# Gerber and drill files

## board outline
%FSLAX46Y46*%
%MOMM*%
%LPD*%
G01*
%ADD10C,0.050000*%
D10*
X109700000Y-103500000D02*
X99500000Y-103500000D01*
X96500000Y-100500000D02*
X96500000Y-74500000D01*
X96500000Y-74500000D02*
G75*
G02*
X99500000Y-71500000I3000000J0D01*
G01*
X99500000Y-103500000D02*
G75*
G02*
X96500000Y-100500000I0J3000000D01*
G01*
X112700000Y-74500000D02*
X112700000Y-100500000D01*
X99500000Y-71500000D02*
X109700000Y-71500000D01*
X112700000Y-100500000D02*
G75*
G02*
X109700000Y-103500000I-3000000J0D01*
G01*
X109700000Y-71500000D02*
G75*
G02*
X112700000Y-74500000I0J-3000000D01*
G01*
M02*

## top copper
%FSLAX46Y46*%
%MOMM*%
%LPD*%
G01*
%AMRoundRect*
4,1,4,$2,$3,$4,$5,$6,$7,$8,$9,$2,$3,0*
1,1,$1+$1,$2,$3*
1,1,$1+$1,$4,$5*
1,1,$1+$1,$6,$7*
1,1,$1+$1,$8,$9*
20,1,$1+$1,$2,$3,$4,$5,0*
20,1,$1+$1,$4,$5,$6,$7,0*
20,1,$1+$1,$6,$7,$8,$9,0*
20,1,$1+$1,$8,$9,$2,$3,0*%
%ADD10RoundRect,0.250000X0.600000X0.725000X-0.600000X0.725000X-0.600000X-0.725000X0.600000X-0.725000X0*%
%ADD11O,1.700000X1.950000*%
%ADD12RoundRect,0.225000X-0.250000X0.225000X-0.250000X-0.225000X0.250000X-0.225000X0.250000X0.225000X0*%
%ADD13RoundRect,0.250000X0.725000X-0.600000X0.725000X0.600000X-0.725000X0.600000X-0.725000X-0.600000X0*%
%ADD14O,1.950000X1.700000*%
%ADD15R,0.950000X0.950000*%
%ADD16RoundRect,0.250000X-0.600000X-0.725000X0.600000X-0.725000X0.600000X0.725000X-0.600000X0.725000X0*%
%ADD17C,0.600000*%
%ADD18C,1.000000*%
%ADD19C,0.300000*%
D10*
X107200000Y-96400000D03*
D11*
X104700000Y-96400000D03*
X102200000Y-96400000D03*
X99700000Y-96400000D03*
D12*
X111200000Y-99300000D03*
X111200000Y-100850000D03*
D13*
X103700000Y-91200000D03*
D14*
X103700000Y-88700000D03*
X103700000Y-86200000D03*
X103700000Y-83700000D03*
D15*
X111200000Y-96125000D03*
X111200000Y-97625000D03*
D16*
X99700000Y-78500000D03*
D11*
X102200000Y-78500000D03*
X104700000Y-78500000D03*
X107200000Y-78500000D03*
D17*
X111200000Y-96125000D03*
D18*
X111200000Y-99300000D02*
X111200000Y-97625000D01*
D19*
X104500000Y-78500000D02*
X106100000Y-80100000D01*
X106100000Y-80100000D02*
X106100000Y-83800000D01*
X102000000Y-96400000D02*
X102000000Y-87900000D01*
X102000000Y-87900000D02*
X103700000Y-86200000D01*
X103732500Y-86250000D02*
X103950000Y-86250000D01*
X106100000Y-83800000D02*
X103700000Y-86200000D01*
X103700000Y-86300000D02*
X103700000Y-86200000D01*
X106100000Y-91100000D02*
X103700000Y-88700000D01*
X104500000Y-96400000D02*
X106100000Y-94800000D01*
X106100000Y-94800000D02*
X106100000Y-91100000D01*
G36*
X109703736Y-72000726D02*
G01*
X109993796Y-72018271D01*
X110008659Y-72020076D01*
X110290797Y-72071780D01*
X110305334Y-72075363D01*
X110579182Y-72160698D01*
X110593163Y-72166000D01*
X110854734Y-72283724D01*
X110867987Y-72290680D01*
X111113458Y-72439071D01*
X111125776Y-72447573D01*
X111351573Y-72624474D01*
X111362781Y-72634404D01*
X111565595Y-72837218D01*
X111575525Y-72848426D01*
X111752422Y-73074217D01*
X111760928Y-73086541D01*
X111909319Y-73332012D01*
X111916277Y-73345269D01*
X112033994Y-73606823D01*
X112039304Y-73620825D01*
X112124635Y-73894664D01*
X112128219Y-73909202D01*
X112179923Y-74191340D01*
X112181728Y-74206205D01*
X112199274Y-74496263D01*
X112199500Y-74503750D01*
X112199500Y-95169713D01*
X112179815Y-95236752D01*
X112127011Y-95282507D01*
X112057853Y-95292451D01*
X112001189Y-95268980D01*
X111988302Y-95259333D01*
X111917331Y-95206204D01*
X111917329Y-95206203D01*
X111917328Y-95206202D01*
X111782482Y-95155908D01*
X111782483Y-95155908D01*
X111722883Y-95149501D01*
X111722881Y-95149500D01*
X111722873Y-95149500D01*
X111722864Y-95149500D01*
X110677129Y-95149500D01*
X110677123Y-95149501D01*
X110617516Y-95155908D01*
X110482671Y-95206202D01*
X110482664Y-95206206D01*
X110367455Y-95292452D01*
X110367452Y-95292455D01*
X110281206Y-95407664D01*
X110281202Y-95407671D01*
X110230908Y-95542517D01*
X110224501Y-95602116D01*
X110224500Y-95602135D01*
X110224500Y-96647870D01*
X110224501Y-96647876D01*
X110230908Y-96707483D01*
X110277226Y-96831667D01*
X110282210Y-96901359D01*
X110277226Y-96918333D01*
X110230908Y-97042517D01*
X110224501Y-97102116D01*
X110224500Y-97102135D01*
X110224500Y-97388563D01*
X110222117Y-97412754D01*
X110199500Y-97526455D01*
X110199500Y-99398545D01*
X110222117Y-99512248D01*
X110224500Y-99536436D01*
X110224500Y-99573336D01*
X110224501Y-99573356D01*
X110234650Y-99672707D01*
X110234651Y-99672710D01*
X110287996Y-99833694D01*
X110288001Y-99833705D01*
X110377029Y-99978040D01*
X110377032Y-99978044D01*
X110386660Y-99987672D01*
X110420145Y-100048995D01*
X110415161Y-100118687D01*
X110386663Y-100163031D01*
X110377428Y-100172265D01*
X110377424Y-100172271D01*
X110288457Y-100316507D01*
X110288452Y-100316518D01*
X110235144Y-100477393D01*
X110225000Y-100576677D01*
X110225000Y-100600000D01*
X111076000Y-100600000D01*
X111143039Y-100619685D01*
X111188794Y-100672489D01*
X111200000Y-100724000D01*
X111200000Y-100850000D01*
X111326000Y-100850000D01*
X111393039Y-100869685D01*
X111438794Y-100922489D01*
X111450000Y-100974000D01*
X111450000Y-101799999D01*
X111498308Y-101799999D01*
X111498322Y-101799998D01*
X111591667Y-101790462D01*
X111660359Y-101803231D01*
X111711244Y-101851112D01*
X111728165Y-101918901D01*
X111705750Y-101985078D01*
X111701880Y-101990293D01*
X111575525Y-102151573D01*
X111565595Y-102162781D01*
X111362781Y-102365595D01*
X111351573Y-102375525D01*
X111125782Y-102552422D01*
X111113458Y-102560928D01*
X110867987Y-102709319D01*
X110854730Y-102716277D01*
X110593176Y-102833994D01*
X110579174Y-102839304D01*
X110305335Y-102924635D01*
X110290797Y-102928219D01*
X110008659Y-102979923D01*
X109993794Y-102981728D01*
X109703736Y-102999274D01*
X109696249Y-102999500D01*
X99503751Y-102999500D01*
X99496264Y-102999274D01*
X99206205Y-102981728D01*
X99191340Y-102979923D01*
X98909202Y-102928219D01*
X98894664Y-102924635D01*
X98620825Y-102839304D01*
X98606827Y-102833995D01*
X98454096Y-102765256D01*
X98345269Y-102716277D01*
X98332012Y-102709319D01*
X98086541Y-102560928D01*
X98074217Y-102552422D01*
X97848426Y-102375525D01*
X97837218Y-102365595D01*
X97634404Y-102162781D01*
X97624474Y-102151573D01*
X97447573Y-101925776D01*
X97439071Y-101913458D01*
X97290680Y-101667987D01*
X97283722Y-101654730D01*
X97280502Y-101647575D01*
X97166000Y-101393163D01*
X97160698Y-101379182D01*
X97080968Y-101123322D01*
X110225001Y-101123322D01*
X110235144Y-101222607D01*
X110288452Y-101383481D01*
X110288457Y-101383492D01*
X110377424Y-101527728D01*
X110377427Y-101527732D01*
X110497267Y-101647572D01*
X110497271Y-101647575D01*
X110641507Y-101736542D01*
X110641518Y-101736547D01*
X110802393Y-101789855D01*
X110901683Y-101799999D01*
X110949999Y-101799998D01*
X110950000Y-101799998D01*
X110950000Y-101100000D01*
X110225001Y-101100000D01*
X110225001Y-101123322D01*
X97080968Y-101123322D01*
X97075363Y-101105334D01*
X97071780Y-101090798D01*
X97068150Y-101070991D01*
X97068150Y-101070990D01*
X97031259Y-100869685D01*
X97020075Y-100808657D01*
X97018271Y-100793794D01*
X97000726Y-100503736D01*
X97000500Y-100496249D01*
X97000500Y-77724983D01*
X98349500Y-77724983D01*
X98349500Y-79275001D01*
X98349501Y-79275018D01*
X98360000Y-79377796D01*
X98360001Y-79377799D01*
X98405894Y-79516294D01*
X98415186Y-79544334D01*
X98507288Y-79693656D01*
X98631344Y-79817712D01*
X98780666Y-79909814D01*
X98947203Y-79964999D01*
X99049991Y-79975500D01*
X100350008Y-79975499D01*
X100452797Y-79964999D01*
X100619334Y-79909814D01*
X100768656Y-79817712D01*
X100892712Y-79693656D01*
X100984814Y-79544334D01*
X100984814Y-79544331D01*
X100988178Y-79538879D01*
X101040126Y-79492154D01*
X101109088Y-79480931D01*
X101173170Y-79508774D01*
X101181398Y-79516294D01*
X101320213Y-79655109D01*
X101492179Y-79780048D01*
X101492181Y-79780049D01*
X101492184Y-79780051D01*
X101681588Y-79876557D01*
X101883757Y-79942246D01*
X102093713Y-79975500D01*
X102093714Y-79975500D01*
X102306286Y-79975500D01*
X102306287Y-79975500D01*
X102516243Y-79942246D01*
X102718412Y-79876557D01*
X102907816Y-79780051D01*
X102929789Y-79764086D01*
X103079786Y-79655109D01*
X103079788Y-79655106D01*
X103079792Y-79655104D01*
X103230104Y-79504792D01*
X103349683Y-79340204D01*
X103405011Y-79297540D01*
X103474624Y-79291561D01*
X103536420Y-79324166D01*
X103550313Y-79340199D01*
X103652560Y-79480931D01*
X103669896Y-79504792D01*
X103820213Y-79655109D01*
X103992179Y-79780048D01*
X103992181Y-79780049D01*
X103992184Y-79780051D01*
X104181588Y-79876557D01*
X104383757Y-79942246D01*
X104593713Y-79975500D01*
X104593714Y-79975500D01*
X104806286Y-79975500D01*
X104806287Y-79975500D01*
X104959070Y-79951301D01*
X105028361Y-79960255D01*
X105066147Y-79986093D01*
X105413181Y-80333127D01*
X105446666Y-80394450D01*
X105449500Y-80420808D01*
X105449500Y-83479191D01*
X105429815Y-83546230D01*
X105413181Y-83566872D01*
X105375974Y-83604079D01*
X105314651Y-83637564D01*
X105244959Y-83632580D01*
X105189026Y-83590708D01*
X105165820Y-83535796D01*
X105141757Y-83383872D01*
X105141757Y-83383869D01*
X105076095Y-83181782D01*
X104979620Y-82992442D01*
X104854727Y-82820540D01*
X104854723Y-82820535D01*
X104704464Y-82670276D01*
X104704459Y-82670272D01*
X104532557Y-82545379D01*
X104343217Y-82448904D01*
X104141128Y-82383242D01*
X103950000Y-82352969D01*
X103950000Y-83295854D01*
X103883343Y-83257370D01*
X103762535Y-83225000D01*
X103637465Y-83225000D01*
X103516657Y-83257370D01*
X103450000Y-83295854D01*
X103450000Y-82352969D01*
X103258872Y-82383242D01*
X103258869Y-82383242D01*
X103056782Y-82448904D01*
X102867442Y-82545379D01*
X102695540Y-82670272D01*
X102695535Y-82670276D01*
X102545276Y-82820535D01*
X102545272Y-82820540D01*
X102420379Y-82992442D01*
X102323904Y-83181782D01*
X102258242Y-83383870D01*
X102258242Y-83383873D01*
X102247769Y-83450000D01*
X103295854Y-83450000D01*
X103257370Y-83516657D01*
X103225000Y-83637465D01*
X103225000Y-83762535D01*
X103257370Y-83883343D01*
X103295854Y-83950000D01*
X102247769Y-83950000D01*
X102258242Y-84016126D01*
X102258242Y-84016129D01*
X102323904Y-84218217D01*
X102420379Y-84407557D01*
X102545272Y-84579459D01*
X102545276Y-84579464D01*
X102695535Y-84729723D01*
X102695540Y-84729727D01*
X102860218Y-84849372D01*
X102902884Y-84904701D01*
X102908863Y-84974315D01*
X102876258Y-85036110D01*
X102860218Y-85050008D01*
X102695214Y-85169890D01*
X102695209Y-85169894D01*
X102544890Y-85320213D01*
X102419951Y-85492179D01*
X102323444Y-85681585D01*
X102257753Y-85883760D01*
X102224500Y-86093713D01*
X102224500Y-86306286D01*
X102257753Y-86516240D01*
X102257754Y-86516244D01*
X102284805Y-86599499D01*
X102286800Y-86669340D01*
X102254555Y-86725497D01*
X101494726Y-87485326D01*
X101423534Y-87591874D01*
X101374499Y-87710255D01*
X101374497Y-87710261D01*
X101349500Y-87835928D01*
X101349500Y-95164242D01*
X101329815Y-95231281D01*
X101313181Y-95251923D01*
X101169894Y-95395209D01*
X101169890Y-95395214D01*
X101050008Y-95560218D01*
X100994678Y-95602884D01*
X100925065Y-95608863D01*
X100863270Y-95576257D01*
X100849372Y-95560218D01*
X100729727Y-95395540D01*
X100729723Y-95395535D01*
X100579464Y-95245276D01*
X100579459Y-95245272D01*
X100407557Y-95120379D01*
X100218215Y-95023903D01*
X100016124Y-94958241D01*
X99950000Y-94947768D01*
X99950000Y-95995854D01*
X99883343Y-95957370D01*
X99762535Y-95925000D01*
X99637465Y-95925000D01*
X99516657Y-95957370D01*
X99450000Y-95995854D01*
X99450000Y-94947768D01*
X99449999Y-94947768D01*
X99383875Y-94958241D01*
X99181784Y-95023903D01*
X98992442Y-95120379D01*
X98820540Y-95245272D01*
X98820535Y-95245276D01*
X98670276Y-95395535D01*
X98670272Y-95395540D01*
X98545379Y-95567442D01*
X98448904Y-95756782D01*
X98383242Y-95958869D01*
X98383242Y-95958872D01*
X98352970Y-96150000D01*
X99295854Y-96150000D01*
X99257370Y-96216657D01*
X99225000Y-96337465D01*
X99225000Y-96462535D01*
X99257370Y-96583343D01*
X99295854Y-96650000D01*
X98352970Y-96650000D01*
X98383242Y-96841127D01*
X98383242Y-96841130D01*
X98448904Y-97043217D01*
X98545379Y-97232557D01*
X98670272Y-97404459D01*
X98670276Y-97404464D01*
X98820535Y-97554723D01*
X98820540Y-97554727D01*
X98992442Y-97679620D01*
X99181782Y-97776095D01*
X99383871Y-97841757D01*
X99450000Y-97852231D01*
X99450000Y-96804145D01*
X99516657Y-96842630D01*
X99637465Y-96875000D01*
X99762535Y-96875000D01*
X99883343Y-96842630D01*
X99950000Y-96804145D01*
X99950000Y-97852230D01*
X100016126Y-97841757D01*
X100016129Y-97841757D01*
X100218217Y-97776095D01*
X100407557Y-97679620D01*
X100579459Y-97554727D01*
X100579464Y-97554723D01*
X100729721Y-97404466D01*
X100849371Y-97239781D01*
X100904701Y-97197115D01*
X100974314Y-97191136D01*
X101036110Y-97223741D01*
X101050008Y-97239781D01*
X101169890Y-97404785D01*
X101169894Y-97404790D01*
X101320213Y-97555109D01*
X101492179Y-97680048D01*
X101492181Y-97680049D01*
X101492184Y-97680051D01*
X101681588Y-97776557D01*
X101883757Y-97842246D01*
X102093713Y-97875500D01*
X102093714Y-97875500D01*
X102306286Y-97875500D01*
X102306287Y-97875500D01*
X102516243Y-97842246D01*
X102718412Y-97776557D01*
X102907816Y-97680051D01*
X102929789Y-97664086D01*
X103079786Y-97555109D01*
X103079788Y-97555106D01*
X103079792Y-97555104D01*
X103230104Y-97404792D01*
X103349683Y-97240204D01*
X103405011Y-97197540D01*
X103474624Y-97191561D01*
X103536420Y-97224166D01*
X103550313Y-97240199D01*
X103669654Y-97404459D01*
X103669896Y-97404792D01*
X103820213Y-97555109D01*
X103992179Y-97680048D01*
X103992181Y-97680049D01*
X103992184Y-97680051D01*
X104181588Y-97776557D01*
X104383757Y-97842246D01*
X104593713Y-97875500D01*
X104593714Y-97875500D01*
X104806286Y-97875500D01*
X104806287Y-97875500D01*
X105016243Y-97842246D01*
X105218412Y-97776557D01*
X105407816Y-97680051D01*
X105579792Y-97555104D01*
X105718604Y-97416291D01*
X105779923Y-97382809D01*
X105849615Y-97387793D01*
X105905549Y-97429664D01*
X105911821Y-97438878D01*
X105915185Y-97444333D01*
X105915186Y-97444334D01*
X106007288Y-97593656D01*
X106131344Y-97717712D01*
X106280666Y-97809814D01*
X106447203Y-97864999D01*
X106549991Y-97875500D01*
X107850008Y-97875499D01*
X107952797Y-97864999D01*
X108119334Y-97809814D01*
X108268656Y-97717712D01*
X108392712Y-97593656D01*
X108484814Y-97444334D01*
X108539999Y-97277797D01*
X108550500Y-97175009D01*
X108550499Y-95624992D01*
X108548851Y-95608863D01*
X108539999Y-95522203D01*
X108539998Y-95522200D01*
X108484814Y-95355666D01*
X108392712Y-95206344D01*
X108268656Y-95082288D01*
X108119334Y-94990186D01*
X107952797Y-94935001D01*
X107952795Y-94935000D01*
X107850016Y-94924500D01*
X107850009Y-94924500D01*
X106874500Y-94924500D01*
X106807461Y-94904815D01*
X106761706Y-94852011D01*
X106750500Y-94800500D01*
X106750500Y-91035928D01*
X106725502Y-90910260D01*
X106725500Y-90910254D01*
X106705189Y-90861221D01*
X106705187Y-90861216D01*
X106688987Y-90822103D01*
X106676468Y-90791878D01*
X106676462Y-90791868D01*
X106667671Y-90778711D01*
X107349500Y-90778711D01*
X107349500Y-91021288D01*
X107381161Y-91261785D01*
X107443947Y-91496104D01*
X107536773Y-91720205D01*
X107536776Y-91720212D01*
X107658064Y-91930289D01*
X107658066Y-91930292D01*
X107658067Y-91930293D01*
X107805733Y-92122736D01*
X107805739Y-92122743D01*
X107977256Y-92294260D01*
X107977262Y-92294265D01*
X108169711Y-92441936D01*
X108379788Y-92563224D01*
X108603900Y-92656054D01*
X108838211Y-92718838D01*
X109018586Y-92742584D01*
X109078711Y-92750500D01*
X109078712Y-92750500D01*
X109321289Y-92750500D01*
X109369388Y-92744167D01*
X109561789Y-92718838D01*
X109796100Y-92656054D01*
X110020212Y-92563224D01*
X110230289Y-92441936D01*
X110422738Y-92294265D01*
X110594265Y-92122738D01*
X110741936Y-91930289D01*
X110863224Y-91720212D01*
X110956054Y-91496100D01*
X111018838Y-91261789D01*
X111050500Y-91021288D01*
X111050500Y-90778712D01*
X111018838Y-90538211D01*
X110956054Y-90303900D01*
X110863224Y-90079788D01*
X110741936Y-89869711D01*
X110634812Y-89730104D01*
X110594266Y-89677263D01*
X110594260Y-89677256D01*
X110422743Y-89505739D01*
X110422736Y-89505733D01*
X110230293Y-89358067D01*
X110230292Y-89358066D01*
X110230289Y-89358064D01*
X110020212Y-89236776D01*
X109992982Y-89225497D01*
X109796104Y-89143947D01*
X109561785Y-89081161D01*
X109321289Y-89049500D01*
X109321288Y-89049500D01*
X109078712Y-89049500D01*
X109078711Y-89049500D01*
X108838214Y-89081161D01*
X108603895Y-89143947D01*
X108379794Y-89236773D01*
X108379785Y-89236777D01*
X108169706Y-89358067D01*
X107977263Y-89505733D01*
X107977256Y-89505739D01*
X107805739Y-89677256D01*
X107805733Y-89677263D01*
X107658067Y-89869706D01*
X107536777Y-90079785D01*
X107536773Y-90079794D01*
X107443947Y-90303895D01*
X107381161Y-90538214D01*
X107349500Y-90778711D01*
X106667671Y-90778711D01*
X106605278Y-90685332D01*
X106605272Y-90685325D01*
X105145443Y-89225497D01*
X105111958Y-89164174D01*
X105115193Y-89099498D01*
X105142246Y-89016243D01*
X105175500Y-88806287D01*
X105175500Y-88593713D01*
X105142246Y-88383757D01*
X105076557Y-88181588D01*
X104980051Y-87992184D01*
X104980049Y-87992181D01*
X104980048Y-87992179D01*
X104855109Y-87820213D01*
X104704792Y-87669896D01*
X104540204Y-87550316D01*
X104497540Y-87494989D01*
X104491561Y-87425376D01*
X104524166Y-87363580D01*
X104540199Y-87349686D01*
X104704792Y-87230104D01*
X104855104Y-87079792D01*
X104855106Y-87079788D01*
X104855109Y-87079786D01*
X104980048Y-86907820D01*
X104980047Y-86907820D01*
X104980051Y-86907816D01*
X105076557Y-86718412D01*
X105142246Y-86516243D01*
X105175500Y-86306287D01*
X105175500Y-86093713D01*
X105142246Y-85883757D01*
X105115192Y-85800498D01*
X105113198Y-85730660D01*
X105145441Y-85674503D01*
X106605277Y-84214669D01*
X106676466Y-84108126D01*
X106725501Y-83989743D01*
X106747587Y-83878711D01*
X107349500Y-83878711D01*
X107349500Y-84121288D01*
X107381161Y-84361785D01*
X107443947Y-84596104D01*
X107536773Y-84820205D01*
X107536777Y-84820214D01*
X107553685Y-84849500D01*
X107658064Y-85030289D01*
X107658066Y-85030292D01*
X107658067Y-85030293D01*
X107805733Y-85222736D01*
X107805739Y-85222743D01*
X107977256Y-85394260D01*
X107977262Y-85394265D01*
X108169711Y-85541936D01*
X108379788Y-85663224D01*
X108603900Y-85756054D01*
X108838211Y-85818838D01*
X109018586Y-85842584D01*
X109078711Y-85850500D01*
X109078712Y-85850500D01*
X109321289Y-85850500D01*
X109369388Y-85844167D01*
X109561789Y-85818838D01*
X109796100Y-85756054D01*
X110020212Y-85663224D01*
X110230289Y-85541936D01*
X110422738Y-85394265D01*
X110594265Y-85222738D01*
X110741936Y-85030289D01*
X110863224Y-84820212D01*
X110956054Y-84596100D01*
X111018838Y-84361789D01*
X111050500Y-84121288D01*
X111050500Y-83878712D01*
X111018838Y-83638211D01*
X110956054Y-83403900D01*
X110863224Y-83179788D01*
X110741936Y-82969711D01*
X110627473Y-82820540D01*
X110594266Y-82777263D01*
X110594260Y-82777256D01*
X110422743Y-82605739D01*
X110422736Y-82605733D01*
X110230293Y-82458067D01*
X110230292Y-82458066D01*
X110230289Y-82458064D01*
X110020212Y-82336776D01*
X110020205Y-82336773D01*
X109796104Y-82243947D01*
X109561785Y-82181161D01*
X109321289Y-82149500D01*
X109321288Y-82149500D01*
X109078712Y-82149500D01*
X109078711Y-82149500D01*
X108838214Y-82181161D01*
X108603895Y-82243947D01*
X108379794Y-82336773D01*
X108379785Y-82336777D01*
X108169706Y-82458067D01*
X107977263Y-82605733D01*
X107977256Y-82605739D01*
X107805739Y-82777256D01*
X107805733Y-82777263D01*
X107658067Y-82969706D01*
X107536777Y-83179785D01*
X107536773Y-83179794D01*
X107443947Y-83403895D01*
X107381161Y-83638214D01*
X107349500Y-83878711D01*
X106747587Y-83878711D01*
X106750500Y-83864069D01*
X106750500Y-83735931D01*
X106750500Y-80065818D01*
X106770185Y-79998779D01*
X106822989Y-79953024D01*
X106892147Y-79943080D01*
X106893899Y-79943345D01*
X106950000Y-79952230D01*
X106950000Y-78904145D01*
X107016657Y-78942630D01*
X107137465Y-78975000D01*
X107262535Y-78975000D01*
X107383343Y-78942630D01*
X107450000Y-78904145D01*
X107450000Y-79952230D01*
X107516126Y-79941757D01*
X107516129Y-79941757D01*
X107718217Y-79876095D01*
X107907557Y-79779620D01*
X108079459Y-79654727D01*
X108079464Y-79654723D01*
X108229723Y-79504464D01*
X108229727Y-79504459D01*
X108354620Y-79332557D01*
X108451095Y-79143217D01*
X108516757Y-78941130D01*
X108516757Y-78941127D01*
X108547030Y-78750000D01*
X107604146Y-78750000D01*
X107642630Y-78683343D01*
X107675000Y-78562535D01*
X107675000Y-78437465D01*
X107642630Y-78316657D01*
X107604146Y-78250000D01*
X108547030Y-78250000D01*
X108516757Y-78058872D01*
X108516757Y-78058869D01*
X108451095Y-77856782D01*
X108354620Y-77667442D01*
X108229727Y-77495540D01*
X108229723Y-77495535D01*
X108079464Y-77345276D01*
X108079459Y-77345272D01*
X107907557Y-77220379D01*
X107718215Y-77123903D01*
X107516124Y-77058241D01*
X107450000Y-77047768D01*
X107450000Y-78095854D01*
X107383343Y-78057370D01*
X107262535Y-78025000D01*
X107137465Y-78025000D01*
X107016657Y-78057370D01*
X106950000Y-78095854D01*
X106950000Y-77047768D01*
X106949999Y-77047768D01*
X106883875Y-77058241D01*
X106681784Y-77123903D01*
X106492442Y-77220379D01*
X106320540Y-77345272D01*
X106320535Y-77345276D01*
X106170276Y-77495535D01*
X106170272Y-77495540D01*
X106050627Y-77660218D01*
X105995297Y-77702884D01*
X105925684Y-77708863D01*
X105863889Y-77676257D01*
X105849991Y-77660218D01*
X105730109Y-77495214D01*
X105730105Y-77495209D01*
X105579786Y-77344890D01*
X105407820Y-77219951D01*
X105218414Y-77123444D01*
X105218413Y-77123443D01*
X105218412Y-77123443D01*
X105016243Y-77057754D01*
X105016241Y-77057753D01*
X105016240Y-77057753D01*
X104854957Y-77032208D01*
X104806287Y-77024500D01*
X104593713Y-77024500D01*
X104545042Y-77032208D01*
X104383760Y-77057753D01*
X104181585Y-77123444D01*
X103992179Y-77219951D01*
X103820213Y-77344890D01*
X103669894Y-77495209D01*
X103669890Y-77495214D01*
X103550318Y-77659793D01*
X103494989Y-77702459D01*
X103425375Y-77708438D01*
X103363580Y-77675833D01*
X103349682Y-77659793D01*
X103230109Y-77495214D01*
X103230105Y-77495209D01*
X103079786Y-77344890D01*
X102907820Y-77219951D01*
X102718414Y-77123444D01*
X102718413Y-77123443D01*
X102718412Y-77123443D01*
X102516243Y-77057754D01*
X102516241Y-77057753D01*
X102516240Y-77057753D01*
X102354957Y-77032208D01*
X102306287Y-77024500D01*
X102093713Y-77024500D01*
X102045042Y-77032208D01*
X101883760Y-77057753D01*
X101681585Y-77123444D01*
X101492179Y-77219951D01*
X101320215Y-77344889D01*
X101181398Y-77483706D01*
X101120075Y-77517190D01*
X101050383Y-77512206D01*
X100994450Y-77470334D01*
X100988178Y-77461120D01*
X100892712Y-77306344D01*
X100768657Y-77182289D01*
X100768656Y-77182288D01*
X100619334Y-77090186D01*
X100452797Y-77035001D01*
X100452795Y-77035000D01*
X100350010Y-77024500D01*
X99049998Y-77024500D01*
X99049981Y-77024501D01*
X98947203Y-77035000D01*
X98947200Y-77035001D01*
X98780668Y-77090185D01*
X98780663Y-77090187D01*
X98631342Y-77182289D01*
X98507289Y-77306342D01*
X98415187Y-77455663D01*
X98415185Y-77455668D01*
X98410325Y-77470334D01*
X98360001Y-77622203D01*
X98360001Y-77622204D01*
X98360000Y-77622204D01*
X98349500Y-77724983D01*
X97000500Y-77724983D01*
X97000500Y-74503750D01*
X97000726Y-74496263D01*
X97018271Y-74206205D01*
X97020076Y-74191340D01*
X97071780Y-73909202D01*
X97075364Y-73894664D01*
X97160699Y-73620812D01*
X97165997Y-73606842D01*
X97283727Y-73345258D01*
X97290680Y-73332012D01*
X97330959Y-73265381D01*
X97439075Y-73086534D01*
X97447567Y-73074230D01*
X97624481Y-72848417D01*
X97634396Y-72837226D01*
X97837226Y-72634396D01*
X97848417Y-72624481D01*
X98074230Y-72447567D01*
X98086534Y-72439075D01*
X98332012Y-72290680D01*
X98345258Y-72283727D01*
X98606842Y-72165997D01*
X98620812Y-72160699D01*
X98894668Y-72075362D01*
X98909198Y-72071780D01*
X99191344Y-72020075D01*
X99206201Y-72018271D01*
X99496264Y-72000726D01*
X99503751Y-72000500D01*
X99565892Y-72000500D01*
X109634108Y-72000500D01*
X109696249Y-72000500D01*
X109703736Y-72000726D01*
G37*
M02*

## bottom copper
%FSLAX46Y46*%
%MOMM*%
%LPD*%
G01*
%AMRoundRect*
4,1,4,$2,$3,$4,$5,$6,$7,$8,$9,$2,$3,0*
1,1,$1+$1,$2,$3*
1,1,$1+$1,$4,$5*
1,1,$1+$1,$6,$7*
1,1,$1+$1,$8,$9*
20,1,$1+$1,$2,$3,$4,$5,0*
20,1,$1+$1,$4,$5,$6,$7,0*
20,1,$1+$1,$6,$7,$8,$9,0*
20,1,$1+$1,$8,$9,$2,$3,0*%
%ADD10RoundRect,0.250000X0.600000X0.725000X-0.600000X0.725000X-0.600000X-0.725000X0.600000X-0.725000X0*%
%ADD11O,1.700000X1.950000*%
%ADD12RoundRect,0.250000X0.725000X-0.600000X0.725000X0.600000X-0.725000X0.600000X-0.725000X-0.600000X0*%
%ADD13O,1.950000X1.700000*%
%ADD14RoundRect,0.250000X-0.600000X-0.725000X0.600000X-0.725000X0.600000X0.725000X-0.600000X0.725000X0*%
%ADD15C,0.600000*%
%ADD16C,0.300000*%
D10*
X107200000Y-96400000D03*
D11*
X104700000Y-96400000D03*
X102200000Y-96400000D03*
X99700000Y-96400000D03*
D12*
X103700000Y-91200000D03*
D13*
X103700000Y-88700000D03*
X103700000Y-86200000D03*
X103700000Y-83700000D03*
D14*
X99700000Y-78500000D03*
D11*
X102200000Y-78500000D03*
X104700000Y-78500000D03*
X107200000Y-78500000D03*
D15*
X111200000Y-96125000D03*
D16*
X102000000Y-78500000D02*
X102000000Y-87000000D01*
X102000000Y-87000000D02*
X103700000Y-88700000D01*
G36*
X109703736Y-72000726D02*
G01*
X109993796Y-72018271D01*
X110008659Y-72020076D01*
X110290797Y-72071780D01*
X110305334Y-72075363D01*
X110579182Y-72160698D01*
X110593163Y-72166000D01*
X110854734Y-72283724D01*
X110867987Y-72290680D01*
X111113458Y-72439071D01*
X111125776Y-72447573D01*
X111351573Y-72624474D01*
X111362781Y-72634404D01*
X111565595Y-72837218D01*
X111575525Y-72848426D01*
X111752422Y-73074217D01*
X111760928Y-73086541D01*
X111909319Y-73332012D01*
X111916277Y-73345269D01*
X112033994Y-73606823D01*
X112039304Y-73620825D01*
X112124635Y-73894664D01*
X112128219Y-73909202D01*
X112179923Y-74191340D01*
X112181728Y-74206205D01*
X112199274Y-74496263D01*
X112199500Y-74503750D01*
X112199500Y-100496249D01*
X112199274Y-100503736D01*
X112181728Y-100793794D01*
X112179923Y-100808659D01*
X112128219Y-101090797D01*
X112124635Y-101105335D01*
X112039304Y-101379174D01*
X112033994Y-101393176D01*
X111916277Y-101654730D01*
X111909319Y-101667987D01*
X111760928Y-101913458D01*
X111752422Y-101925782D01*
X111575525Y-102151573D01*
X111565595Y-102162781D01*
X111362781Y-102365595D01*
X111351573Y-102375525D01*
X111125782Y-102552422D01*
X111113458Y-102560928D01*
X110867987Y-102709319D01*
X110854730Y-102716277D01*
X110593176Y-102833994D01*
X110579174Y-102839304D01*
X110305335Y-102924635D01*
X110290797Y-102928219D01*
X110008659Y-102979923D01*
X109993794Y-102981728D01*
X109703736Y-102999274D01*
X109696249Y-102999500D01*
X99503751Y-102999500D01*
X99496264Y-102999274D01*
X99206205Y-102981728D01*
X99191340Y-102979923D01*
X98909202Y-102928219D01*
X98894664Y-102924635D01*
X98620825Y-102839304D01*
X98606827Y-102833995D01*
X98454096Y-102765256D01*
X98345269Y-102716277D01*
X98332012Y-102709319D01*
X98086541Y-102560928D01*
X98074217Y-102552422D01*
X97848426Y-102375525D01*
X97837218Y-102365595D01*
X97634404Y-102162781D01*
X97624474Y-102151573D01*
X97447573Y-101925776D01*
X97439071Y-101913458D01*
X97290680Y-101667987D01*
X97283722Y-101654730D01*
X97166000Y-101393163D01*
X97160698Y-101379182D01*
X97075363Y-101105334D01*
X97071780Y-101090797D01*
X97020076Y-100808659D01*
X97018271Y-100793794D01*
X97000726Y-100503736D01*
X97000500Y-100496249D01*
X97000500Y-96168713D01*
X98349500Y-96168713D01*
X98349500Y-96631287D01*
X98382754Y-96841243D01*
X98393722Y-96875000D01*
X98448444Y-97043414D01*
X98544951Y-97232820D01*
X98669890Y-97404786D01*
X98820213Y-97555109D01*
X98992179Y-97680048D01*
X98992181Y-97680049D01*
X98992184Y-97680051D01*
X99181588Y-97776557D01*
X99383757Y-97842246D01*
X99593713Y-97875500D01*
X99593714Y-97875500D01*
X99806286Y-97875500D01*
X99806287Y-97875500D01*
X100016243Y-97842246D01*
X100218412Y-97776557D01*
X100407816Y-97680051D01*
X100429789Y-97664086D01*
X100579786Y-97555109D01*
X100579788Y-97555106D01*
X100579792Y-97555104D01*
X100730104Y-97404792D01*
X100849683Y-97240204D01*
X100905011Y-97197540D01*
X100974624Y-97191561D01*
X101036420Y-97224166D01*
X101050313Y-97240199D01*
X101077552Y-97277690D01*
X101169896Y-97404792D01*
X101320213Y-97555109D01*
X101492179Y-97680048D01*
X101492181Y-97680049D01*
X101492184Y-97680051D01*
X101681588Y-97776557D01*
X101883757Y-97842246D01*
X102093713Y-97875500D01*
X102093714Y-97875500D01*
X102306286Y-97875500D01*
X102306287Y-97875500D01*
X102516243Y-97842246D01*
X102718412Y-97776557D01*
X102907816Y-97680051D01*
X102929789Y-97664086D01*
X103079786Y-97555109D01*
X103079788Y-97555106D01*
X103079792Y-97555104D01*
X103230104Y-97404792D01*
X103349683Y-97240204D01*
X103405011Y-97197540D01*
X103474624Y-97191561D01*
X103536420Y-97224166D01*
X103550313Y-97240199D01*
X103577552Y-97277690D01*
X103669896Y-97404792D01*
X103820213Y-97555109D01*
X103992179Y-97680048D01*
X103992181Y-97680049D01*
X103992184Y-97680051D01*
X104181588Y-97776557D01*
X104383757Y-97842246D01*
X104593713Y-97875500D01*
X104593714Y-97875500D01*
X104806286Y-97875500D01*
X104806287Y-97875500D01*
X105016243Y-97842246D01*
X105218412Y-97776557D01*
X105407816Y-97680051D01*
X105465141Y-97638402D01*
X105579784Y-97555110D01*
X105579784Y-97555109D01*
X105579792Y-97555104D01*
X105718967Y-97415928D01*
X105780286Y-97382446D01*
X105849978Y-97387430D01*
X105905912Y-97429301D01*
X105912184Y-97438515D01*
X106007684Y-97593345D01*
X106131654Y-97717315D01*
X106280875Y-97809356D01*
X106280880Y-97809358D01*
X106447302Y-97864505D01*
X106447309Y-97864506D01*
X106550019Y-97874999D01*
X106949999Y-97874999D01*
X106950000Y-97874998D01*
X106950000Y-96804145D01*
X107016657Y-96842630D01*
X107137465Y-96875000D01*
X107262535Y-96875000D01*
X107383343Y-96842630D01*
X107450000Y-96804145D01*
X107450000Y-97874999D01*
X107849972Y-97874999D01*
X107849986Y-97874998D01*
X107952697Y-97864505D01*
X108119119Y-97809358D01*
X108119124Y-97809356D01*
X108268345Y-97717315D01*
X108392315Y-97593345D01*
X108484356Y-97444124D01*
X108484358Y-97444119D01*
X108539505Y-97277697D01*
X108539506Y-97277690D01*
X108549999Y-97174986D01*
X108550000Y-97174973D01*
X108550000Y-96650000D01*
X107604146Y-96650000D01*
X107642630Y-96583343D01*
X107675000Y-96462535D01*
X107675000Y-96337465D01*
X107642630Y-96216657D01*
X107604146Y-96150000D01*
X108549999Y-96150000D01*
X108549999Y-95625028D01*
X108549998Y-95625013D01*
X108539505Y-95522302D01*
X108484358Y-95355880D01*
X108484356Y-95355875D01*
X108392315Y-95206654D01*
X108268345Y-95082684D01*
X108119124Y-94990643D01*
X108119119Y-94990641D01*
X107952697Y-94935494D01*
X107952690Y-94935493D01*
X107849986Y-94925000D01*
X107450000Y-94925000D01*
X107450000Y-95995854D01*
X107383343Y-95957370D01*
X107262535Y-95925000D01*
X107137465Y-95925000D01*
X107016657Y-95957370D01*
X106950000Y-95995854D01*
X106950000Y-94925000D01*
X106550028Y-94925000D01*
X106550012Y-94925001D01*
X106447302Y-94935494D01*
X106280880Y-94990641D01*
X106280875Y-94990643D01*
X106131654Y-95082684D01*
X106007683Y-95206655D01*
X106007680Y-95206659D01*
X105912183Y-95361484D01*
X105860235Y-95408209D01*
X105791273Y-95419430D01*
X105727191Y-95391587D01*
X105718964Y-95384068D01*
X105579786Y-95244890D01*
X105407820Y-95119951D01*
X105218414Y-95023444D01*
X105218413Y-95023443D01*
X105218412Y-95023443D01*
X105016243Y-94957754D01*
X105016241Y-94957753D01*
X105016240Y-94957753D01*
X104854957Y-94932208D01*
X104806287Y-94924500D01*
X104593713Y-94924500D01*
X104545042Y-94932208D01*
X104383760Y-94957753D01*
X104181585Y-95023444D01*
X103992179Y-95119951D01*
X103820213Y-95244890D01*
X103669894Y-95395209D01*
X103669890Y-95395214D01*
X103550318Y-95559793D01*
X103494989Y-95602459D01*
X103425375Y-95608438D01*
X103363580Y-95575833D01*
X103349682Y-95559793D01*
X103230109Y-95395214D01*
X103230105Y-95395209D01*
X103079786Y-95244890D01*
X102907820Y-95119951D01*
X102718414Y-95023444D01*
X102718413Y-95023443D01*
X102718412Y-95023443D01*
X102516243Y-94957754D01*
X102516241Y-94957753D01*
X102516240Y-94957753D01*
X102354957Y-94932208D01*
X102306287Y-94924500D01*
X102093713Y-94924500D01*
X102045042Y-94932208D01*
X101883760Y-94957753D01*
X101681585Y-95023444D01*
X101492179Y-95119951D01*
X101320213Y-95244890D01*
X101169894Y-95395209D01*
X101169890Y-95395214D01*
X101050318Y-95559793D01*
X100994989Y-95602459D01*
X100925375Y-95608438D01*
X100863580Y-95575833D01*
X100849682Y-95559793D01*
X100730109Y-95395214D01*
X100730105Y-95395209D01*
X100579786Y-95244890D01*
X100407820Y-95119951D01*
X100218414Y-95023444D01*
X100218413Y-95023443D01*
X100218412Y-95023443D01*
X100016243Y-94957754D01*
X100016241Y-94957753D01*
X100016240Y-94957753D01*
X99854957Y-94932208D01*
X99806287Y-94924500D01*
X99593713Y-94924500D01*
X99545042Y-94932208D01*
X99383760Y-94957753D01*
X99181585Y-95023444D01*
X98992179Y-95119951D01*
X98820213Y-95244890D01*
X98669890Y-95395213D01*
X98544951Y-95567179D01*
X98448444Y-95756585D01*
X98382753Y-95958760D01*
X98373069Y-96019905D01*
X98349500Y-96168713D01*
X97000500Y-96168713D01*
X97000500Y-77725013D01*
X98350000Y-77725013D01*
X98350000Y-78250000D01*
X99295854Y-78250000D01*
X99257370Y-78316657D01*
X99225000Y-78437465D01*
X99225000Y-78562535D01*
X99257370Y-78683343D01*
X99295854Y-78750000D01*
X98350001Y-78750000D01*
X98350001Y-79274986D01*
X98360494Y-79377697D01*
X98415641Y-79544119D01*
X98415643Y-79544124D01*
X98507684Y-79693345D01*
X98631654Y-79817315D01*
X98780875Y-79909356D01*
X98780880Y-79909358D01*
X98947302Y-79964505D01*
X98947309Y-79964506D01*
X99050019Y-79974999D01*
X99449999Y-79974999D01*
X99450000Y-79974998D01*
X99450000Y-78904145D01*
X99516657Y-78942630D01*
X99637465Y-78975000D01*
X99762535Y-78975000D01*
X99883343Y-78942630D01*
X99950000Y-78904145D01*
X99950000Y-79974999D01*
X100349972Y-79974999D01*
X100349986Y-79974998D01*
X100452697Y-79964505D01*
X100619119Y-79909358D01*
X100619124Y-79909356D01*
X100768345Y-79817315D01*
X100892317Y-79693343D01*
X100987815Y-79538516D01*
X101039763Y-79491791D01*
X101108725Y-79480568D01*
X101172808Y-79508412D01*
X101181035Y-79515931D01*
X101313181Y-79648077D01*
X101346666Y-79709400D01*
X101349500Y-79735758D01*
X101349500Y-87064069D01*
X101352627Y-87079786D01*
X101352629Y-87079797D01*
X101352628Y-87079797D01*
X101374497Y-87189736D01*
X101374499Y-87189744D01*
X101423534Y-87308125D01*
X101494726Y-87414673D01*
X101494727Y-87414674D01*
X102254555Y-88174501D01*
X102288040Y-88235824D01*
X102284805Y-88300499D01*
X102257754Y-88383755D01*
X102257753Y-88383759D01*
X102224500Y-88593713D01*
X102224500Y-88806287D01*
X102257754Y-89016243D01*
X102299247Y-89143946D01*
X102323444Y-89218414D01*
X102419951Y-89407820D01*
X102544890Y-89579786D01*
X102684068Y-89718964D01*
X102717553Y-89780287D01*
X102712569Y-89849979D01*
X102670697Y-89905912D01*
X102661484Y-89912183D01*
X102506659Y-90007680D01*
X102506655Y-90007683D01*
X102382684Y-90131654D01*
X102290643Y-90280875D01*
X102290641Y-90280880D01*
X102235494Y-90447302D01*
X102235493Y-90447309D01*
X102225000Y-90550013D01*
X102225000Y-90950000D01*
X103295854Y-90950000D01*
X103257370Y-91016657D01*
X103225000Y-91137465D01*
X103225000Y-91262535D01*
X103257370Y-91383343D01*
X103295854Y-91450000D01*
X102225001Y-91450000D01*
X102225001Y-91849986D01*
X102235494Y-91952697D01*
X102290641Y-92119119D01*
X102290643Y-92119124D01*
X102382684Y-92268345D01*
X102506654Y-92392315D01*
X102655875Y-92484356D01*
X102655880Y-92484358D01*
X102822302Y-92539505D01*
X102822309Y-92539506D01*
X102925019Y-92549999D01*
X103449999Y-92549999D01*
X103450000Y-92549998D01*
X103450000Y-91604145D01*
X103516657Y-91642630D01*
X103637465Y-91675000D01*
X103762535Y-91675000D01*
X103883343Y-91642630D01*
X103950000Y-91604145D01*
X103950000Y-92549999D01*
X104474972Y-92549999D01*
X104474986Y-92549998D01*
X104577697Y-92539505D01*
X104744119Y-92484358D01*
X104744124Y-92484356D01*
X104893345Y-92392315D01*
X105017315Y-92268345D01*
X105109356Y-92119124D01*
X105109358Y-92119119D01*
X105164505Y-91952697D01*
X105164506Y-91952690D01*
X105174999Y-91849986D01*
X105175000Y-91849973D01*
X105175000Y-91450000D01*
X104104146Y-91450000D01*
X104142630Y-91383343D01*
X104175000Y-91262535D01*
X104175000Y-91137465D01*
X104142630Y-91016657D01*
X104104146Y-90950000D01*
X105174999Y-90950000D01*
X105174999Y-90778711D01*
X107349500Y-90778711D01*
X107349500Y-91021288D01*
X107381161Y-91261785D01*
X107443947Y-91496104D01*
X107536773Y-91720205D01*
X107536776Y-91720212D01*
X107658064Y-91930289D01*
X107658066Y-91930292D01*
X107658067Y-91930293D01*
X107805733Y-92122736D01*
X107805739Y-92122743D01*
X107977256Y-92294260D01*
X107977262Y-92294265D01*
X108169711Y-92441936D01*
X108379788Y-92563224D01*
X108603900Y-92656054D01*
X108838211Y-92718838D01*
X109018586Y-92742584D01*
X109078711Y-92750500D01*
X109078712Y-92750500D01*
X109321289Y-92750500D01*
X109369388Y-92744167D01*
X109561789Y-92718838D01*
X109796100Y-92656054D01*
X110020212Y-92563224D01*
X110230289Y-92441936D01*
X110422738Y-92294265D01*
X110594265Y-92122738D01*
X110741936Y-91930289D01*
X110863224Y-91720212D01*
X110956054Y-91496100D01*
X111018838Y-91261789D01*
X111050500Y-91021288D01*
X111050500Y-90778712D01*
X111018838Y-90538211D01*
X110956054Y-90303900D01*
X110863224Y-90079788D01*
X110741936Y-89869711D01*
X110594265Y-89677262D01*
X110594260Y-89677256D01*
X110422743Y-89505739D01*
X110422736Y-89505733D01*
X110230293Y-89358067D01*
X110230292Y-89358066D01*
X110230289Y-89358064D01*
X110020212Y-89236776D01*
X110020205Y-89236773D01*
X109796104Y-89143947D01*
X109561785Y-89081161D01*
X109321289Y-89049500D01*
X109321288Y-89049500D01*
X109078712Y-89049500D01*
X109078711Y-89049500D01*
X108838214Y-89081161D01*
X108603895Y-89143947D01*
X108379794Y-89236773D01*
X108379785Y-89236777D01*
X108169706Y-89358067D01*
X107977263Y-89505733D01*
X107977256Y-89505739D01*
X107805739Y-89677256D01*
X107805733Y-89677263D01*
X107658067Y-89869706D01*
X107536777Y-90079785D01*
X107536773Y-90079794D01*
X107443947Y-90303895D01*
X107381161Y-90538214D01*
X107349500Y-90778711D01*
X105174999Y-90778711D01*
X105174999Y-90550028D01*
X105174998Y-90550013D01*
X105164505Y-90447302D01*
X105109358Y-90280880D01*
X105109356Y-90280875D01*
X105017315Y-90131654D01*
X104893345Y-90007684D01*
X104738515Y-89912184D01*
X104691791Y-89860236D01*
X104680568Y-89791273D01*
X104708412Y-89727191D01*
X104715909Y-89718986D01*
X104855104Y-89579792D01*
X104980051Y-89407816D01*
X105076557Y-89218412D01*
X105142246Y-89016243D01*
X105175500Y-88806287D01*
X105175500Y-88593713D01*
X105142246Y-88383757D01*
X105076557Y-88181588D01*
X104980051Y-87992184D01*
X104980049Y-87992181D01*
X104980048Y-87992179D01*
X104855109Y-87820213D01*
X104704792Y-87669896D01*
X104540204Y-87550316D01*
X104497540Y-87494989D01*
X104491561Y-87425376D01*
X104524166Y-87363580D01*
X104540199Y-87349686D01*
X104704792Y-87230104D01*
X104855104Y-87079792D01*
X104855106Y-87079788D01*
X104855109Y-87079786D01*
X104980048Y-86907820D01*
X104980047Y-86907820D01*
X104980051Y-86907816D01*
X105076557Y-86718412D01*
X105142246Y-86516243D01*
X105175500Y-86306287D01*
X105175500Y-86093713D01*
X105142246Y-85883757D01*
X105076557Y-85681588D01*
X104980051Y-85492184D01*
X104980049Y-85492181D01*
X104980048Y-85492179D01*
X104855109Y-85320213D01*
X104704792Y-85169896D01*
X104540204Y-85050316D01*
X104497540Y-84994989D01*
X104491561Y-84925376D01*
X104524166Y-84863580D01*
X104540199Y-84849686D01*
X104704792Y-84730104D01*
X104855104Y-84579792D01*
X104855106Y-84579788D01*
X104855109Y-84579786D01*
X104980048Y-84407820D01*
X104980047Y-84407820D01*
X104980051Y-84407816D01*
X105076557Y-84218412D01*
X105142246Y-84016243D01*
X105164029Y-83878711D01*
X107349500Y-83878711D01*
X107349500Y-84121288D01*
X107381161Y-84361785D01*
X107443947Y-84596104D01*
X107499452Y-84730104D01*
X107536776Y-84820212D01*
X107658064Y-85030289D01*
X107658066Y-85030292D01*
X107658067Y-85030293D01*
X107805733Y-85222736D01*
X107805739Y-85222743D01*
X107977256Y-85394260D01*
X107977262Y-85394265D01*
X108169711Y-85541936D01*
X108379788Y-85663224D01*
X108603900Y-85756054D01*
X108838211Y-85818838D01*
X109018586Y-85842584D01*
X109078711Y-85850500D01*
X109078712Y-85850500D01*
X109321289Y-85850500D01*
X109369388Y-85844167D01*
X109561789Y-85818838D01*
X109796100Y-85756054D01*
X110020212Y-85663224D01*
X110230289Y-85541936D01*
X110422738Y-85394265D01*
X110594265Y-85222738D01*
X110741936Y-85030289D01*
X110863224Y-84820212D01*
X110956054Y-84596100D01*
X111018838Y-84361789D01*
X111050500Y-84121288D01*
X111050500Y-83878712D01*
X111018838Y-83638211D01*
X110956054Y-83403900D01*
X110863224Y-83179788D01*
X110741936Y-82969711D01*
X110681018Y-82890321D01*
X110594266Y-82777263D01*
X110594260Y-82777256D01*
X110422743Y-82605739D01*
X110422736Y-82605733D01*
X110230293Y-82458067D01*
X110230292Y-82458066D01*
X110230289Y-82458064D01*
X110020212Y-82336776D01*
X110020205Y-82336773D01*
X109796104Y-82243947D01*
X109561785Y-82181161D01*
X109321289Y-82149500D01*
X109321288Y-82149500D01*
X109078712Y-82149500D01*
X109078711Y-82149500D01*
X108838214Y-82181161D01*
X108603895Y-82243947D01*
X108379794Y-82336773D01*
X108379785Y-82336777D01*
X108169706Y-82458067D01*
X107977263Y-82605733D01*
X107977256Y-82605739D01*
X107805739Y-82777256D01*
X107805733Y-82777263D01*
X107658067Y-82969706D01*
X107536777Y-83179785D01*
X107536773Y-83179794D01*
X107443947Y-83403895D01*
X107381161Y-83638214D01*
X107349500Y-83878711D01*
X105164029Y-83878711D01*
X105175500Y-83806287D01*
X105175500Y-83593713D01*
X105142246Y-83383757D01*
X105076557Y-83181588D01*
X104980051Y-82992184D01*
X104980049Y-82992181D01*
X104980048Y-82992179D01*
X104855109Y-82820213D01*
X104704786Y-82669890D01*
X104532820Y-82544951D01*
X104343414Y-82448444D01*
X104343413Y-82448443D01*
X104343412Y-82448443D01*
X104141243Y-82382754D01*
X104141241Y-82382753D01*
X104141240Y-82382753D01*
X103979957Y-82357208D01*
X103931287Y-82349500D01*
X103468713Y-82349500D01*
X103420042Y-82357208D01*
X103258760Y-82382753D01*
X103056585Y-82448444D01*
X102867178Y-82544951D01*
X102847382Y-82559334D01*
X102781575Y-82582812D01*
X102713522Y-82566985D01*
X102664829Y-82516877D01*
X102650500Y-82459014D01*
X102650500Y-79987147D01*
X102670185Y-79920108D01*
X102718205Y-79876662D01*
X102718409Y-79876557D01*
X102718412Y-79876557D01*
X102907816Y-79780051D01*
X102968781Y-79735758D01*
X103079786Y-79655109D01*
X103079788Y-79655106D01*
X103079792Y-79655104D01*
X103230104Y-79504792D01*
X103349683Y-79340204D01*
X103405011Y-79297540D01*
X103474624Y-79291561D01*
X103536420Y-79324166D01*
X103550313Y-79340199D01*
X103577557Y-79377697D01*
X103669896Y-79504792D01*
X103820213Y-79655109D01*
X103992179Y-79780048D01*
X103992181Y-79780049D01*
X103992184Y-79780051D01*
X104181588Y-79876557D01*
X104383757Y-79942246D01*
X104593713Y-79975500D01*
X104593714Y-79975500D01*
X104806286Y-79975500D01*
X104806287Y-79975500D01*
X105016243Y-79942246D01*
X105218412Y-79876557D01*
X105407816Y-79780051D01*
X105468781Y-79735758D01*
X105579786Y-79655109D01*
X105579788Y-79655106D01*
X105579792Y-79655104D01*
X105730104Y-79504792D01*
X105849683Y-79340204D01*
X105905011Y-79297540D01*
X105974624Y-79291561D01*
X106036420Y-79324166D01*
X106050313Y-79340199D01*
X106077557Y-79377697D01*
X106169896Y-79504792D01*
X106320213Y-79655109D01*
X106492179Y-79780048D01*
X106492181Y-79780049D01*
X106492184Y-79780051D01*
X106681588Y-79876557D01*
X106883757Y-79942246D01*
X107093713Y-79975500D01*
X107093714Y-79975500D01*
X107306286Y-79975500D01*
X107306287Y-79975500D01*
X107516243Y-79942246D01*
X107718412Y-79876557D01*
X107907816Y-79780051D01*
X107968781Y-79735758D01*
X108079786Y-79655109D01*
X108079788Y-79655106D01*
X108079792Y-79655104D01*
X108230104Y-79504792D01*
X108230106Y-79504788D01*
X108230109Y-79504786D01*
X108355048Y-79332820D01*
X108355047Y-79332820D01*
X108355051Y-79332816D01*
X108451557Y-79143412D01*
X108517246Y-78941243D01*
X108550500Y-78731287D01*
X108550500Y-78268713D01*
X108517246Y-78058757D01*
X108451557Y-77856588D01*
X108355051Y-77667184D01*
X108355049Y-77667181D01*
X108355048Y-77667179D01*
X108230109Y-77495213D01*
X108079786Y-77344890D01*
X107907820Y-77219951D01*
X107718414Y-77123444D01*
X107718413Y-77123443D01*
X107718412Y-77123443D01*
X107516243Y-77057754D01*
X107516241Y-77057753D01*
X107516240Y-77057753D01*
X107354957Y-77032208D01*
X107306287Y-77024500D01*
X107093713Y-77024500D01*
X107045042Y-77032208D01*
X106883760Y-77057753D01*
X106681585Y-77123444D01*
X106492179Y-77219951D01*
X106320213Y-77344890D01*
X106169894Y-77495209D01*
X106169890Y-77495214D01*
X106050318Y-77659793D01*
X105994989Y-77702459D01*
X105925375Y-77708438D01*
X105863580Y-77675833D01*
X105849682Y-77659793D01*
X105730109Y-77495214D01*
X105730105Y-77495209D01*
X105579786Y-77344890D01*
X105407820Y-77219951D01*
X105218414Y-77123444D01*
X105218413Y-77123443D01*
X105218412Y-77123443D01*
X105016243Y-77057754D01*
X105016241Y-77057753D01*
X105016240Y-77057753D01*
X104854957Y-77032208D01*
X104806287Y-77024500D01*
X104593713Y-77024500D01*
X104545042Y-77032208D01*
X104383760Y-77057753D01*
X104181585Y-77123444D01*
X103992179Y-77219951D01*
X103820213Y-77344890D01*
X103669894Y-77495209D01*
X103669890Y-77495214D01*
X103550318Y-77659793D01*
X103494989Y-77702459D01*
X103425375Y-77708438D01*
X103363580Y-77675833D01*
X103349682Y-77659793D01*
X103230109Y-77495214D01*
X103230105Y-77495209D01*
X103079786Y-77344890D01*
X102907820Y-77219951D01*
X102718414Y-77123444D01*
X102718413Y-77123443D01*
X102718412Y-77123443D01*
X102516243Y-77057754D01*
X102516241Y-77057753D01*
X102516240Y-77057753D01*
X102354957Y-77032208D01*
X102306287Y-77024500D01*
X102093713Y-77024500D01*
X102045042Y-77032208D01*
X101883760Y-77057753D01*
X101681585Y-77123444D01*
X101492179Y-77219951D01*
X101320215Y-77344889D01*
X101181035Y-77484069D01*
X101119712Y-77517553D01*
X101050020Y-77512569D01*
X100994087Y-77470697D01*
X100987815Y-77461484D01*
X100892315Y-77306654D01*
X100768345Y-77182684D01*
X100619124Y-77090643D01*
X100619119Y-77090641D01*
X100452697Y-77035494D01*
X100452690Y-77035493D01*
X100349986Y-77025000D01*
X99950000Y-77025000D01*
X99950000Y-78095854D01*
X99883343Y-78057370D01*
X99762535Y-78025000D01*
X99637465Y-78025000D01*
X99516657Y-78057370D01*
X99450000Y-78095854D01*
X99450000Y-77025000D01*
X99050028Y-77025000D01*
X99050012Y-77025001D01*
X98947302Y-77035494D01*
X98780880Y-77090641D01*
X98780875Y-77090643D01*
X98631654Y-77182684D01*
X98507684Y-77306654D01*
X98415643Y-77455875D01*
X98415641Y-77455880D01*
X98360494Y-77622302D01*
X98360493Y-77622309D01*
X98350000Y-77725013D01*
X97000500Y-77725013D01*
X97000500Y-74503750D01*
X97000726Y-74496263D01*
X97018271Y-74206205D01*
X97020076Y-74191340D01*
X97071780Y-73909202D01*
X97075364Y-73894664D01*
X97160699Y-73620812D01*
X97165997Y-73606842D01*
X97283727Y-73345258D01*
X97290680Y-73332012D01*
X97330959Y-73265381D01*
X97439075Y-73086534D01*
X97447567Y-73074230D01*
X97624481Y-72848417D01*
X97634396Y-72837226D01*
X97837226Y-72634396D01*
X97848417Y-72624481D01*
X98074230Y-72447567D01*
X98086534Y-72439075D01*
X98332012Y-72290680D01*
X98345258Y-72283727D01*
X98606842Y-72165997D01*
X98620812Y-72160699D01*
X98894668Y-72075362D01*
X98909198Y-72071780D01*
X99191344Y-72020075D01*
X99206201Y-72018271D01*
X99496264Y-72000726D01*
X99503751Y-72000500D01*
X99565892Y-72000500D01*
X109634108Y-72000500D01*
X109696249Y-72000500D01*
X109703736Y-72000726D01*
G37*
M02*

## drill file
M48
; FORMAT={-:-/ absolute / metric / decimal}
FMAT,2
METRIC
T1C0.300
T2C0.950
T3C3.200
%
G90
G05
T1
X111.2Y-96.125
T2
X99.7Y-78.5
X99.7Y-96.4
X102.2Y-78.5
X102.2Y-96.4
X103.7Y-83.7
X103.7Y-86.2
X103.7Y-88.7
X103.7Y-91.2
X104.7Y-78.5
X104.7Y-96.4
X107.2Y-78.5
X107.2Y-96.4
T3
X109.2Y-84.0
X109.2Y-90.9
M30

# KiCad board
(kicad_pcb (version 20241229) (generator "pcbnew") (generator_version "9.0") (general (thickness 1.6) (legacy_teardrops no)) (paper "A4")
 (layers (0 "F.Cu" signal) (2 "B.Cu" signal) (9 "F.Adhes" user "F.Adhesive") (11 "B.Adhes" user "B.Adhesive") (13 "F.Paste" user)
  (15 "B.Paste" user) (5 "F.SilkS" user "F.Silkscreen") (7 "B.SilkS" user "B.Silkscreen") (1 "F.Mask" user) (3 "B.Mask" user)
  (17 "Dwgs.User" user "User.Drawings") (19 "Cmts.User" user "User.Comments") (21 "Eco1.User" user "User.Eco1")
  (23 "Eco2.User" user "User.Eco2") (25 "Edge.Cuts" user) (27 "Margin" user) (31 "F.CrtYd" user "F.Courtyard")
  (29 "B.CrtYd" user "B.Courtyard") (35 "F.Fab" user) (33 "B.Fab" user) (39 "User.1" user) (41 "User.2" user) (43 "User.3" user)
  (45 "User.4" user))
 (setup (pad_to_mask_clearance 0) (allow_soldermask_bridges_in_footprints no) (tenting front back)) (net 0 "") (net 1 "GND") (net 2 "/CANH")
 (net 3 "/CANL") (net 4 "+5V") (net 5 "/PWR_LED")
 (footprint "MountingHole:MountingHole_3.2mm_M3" (layer "F.Cu") (at 109.2 90.9)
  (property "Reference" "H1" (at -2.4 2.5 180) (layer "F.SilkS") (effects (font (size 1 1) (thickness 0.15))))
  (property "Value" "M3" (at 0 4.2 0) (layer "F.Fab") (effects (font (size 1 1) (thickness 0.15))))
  (pad "" np_thru_hole circle (at 0 0) (size 3.2 3.2) (drill 3.2) (layers "*.Cu" "*.Mask")))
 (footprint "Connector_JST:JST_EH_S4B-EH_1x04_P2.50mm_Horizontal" (layer "F.Cu") (at 107.2 96.4 180)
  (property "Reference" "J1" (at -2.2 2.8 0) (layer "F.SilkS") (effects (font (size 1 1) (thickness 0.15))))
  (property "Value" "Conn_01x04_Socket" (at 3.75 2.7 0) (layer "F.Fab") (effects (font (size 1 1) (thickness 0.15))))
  (pad "1" thru_hole roundrect (at 0 0 180) (size 1.7 1.95) (drill 0.95) (layers "*.Cu" "*.Mask") (remove_unused_layers no)
   (roundrect_rratio 0.147059) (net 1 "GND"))
  (pad "2" thru_hole oval (at 2.5 0 180) (size 1.7 1.95) (drill 0.95) (layers "*.Cu" "*.Mask") (remove_unused_layers no) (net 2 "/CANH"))
  (pad "3" thru_hole oval (at 5 0 180) (size 1.7 1.95) (drill 0.95) (layers "*.Cu" "*.Mask") (remove_unused_layers no) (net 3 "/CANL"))
  (pad "4" thru_hole oval (at 7.5 0 180) (size 1.7 1.95) (drill 0.95) (layers "*.Cu" "*.Mask") (remove_unused_layers no) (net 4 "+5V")))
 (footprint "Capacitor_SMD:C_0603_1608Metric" (layer "F.Cu") (at 111.2 100.075 -90)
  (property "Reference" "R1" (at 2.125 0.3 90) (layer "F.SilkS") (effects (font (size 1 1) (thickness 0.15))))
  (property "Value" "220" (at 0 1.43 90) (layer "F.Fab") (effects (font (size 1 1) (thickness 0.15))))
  (pad "1" smd roundrect (at -0.775 0 270) (size 0.9 0.95) (layers "F.Cu" "F.Mask" "F.Paste") (roundrect_rratio 0.25) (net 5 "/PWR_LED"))
  (pad "2" smd roundrect (at 0.775 0 270) (size 0.9 0.95) (layers "F.Cu" "F.Mask" "F.Paste") (roundrect_rratio 0.25) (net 4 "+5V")))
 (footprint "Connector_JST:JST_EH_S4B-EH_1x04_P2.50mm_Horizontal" (layer "F.Cu") (at 103.7 91.2 90)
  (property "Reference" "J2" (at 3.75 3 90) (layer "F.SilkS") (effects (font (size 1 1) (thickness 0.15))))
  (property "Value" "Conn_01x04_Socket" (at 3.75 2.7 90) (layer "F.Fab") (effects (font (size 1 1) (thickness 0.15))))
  (pad "1" thru_hole roundrect (at 0 0 90) (size 1.7 1.95) (drill 0.95) (layers "*.Cu" "*.Mask") (remove_unused_layers no)
   (roundrect_rratio 0.147059) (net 1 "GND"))
  (pad "2" thru_hole oval (at 2.5 0 90) (size 1.7 1.95) (drill 0.95) (layers "*.Cu" "*.Mask") (remove_unused_layers no) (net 2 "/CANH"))
  (pad "3" thru_hole oval (at 5 0 90) (size 1.7 1.95) (drill 0.95) (layers "*.Cu" "*.Mask") (remove_unused_layers no) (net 3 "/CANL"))
  (pad "4" thru_hole oval (at 7.5 0 90) (size 1.7 1.95) (drill 0.95) (layers "*.Cu" "*.Mask") (remove_unused_layers no) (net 4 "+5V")))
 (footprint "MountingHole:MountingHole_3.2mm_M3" (layer "F.Cu") (at 109.2 84)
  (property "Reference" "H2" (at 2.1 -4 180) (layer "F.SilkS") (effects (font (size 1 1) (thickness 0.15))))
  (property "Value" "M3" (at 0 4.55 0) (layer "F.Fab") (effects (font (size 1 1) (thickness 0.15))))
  (pad "" np_thru_hole circle (at 0 0) (size 3.2 3.2) (drill 3.2) (layers "*.Cu" "*.Mask")))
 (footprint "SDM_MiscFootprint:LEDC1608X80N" (layer "F.Cu") (at 111.2 96.875 -90)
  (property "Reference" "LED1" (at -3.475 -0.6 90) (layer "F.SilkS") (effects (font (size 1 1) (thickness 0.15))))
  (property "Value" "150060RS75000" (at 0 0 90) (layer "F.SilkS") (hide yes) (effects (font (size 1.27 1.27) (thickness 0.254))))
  (pad "1" smd rect (at -0.75 0) (size 0.95 0.95) (layers "F.Cu" "F.Mask" "F.Paste") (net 1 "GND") (thermal_bridge_angle 45))
  (pad "2" smd rect (at 0.75 0) (size 0.95 0.95) (layers "F.Cu" "F.Mask" "F.Paste") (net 5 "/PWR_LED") (thermal_bridge_angle 45)))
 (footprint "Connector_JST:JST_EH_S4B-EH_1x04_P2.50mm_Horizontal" (layer "F.Cu") (at 99.7 78.5)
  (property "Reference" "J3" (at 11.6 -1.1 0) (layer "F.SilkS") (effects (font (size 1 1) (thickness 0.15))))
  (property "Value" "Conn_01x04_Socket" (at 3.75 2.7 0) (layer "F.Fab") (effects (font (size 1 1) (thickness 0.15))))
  (pad "1" thru_hole roundrect (at 0 0) (size 1.7 1.95) (drill 0.95) (layers "*.Cu" "*.Mask") (remove_unused_layers no)
   (roundrect_rratio 0.147059) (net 1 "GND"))
  (pad "2" thru_hole oval (at 2.5 0) (size 1.7 1.95) (drill 0.95) (layers "*.Cu" "*.Mask") (remove_unused_layers no) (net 2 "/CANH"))
  (pad "3" thru_hole oval (at 5 0) (size 1.7 1.95) (drill 0.95) (layers "*.Cu" "*.Mask") (remove_unused_layers no) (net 3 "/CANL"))
  (pad "4" thru_hole oval (at 7.5 0) (size 1.7 1.95) (drill 0.95) (layers "*.Cu" "*.Mask") (remove_unused_layers no) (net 4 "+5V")))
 (gr_line (start 109.7 103.5) (end 99.5 103.5) (stroke (width 0.05) (type default)) (layer "Edge.Cuts"))
 (gr_line (start 96.5 100.5) (end 96.5 74.5) (stroke (width 0.05) (type default)) (layer "Edge.Cuts"))
 (gr_arc (start 96.5 74.5) (mid 97.37868 72.37868) (end 99.5 71.5) (stroke (width 0.05) (type default)) (layer "Edge.Cuts"))
 (gr_arc (start 99.5 103.5) (mid 97.37868 102.62132) (end 96.5 100.5) (stroke (width 0.05) (type default)) (layer "Edge.Cuts"))
 (gr_line (start 112.7 74.5) (end 112.7 100.5) (stroke (width 0.05) (type default)) (layer "Edge.Cuts"))
 (gr_line (start 99.5 71.5) (end 109.7 71.5) (stroke (width 0.05) (type default)) (layer "Edge.Cuts"))
 (gr_arc (start 112.7 100.5) (mid 111.82132 102.62132) (end 109.7 103.5) (stroke (width 0.05) (type default)) (layer "Edge.Cuts"))
 (gr_arc (start 109.7 71.5) (mid 111.82132 72.37868) (end 112.7 74.5) (stroke (width 0.05) (type default)) (layer "Edge.Cuts"))
 (via (at 111.2 96.125) (size 0.6) (drill 0.3) (layers "F.Cu" "B.Cu") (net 1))
 (segment (start 111.2 99.3) (end 111.2 97.625) (width 1) (layer "F.Cu") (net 5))
 (segment (start 104.5 78.5) (end 106.1 80.1) (width 0.3) (layer "F.Cu") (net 3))
 (segment (start 106.1 80.1) (end 106.1 83.8) (width 0.3) (layer "F.Cu") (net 3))
 (segment (start 102 96.4) (end 102 87.9) (width 0.3) (layer "F.Cu") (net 3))
 (segment (start 102 87.9) (end 103.7 86.2) (width 0.3) (layer "F.Cu") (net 3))
 (segment (start 103.7325 86.25) (end 103.95 86.25) (width 0.3) (layer "F.Cu") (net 3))
 (segment (start 106.1 83.8) (end 103.7 86.2) (width 0.3) (layer "F.Cu") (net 3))
 (segment (start 103.7 86.3) (end 103.7 86.2) (width 0.3) (layer "F.Cu") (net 3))
 (segment (start 106.1 91.1) (end 103.7 88.7) (width 0.3) (layer "F.Cu") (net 2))
 (segment (start 104.5 96.4) (end 106.1 94.8) (width 0.3) (layer "F.Cu") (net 2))
 (segment (start 106.1 94.8) (end 106.1 91.1) (width 0.3) (layer "F.Cu") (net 2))
 (segment (start 102 78.5) (end 102 87) (width 0.3) (layer "B.Cu") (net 2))
 (segment (start 102 87) (end 103.7 88.7) (width 0.3) (layer "B.Cu") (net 2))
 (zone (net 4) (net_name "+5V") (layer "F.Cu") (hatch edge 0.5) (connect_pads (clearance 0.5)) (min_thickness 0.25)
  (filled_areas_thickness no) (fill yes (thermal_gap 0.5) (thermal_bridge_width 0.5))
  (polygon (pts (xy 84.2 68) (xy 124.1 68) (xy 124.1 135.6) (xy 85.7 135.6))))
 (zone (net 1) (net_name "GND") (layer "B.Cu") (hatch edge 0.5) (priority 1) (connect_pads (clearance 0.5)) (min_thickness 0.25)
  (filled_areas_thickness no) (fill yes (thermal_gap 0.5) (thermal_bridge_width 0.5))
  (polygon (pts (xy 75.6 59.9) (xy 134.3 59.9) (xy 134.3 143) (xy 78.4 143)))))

